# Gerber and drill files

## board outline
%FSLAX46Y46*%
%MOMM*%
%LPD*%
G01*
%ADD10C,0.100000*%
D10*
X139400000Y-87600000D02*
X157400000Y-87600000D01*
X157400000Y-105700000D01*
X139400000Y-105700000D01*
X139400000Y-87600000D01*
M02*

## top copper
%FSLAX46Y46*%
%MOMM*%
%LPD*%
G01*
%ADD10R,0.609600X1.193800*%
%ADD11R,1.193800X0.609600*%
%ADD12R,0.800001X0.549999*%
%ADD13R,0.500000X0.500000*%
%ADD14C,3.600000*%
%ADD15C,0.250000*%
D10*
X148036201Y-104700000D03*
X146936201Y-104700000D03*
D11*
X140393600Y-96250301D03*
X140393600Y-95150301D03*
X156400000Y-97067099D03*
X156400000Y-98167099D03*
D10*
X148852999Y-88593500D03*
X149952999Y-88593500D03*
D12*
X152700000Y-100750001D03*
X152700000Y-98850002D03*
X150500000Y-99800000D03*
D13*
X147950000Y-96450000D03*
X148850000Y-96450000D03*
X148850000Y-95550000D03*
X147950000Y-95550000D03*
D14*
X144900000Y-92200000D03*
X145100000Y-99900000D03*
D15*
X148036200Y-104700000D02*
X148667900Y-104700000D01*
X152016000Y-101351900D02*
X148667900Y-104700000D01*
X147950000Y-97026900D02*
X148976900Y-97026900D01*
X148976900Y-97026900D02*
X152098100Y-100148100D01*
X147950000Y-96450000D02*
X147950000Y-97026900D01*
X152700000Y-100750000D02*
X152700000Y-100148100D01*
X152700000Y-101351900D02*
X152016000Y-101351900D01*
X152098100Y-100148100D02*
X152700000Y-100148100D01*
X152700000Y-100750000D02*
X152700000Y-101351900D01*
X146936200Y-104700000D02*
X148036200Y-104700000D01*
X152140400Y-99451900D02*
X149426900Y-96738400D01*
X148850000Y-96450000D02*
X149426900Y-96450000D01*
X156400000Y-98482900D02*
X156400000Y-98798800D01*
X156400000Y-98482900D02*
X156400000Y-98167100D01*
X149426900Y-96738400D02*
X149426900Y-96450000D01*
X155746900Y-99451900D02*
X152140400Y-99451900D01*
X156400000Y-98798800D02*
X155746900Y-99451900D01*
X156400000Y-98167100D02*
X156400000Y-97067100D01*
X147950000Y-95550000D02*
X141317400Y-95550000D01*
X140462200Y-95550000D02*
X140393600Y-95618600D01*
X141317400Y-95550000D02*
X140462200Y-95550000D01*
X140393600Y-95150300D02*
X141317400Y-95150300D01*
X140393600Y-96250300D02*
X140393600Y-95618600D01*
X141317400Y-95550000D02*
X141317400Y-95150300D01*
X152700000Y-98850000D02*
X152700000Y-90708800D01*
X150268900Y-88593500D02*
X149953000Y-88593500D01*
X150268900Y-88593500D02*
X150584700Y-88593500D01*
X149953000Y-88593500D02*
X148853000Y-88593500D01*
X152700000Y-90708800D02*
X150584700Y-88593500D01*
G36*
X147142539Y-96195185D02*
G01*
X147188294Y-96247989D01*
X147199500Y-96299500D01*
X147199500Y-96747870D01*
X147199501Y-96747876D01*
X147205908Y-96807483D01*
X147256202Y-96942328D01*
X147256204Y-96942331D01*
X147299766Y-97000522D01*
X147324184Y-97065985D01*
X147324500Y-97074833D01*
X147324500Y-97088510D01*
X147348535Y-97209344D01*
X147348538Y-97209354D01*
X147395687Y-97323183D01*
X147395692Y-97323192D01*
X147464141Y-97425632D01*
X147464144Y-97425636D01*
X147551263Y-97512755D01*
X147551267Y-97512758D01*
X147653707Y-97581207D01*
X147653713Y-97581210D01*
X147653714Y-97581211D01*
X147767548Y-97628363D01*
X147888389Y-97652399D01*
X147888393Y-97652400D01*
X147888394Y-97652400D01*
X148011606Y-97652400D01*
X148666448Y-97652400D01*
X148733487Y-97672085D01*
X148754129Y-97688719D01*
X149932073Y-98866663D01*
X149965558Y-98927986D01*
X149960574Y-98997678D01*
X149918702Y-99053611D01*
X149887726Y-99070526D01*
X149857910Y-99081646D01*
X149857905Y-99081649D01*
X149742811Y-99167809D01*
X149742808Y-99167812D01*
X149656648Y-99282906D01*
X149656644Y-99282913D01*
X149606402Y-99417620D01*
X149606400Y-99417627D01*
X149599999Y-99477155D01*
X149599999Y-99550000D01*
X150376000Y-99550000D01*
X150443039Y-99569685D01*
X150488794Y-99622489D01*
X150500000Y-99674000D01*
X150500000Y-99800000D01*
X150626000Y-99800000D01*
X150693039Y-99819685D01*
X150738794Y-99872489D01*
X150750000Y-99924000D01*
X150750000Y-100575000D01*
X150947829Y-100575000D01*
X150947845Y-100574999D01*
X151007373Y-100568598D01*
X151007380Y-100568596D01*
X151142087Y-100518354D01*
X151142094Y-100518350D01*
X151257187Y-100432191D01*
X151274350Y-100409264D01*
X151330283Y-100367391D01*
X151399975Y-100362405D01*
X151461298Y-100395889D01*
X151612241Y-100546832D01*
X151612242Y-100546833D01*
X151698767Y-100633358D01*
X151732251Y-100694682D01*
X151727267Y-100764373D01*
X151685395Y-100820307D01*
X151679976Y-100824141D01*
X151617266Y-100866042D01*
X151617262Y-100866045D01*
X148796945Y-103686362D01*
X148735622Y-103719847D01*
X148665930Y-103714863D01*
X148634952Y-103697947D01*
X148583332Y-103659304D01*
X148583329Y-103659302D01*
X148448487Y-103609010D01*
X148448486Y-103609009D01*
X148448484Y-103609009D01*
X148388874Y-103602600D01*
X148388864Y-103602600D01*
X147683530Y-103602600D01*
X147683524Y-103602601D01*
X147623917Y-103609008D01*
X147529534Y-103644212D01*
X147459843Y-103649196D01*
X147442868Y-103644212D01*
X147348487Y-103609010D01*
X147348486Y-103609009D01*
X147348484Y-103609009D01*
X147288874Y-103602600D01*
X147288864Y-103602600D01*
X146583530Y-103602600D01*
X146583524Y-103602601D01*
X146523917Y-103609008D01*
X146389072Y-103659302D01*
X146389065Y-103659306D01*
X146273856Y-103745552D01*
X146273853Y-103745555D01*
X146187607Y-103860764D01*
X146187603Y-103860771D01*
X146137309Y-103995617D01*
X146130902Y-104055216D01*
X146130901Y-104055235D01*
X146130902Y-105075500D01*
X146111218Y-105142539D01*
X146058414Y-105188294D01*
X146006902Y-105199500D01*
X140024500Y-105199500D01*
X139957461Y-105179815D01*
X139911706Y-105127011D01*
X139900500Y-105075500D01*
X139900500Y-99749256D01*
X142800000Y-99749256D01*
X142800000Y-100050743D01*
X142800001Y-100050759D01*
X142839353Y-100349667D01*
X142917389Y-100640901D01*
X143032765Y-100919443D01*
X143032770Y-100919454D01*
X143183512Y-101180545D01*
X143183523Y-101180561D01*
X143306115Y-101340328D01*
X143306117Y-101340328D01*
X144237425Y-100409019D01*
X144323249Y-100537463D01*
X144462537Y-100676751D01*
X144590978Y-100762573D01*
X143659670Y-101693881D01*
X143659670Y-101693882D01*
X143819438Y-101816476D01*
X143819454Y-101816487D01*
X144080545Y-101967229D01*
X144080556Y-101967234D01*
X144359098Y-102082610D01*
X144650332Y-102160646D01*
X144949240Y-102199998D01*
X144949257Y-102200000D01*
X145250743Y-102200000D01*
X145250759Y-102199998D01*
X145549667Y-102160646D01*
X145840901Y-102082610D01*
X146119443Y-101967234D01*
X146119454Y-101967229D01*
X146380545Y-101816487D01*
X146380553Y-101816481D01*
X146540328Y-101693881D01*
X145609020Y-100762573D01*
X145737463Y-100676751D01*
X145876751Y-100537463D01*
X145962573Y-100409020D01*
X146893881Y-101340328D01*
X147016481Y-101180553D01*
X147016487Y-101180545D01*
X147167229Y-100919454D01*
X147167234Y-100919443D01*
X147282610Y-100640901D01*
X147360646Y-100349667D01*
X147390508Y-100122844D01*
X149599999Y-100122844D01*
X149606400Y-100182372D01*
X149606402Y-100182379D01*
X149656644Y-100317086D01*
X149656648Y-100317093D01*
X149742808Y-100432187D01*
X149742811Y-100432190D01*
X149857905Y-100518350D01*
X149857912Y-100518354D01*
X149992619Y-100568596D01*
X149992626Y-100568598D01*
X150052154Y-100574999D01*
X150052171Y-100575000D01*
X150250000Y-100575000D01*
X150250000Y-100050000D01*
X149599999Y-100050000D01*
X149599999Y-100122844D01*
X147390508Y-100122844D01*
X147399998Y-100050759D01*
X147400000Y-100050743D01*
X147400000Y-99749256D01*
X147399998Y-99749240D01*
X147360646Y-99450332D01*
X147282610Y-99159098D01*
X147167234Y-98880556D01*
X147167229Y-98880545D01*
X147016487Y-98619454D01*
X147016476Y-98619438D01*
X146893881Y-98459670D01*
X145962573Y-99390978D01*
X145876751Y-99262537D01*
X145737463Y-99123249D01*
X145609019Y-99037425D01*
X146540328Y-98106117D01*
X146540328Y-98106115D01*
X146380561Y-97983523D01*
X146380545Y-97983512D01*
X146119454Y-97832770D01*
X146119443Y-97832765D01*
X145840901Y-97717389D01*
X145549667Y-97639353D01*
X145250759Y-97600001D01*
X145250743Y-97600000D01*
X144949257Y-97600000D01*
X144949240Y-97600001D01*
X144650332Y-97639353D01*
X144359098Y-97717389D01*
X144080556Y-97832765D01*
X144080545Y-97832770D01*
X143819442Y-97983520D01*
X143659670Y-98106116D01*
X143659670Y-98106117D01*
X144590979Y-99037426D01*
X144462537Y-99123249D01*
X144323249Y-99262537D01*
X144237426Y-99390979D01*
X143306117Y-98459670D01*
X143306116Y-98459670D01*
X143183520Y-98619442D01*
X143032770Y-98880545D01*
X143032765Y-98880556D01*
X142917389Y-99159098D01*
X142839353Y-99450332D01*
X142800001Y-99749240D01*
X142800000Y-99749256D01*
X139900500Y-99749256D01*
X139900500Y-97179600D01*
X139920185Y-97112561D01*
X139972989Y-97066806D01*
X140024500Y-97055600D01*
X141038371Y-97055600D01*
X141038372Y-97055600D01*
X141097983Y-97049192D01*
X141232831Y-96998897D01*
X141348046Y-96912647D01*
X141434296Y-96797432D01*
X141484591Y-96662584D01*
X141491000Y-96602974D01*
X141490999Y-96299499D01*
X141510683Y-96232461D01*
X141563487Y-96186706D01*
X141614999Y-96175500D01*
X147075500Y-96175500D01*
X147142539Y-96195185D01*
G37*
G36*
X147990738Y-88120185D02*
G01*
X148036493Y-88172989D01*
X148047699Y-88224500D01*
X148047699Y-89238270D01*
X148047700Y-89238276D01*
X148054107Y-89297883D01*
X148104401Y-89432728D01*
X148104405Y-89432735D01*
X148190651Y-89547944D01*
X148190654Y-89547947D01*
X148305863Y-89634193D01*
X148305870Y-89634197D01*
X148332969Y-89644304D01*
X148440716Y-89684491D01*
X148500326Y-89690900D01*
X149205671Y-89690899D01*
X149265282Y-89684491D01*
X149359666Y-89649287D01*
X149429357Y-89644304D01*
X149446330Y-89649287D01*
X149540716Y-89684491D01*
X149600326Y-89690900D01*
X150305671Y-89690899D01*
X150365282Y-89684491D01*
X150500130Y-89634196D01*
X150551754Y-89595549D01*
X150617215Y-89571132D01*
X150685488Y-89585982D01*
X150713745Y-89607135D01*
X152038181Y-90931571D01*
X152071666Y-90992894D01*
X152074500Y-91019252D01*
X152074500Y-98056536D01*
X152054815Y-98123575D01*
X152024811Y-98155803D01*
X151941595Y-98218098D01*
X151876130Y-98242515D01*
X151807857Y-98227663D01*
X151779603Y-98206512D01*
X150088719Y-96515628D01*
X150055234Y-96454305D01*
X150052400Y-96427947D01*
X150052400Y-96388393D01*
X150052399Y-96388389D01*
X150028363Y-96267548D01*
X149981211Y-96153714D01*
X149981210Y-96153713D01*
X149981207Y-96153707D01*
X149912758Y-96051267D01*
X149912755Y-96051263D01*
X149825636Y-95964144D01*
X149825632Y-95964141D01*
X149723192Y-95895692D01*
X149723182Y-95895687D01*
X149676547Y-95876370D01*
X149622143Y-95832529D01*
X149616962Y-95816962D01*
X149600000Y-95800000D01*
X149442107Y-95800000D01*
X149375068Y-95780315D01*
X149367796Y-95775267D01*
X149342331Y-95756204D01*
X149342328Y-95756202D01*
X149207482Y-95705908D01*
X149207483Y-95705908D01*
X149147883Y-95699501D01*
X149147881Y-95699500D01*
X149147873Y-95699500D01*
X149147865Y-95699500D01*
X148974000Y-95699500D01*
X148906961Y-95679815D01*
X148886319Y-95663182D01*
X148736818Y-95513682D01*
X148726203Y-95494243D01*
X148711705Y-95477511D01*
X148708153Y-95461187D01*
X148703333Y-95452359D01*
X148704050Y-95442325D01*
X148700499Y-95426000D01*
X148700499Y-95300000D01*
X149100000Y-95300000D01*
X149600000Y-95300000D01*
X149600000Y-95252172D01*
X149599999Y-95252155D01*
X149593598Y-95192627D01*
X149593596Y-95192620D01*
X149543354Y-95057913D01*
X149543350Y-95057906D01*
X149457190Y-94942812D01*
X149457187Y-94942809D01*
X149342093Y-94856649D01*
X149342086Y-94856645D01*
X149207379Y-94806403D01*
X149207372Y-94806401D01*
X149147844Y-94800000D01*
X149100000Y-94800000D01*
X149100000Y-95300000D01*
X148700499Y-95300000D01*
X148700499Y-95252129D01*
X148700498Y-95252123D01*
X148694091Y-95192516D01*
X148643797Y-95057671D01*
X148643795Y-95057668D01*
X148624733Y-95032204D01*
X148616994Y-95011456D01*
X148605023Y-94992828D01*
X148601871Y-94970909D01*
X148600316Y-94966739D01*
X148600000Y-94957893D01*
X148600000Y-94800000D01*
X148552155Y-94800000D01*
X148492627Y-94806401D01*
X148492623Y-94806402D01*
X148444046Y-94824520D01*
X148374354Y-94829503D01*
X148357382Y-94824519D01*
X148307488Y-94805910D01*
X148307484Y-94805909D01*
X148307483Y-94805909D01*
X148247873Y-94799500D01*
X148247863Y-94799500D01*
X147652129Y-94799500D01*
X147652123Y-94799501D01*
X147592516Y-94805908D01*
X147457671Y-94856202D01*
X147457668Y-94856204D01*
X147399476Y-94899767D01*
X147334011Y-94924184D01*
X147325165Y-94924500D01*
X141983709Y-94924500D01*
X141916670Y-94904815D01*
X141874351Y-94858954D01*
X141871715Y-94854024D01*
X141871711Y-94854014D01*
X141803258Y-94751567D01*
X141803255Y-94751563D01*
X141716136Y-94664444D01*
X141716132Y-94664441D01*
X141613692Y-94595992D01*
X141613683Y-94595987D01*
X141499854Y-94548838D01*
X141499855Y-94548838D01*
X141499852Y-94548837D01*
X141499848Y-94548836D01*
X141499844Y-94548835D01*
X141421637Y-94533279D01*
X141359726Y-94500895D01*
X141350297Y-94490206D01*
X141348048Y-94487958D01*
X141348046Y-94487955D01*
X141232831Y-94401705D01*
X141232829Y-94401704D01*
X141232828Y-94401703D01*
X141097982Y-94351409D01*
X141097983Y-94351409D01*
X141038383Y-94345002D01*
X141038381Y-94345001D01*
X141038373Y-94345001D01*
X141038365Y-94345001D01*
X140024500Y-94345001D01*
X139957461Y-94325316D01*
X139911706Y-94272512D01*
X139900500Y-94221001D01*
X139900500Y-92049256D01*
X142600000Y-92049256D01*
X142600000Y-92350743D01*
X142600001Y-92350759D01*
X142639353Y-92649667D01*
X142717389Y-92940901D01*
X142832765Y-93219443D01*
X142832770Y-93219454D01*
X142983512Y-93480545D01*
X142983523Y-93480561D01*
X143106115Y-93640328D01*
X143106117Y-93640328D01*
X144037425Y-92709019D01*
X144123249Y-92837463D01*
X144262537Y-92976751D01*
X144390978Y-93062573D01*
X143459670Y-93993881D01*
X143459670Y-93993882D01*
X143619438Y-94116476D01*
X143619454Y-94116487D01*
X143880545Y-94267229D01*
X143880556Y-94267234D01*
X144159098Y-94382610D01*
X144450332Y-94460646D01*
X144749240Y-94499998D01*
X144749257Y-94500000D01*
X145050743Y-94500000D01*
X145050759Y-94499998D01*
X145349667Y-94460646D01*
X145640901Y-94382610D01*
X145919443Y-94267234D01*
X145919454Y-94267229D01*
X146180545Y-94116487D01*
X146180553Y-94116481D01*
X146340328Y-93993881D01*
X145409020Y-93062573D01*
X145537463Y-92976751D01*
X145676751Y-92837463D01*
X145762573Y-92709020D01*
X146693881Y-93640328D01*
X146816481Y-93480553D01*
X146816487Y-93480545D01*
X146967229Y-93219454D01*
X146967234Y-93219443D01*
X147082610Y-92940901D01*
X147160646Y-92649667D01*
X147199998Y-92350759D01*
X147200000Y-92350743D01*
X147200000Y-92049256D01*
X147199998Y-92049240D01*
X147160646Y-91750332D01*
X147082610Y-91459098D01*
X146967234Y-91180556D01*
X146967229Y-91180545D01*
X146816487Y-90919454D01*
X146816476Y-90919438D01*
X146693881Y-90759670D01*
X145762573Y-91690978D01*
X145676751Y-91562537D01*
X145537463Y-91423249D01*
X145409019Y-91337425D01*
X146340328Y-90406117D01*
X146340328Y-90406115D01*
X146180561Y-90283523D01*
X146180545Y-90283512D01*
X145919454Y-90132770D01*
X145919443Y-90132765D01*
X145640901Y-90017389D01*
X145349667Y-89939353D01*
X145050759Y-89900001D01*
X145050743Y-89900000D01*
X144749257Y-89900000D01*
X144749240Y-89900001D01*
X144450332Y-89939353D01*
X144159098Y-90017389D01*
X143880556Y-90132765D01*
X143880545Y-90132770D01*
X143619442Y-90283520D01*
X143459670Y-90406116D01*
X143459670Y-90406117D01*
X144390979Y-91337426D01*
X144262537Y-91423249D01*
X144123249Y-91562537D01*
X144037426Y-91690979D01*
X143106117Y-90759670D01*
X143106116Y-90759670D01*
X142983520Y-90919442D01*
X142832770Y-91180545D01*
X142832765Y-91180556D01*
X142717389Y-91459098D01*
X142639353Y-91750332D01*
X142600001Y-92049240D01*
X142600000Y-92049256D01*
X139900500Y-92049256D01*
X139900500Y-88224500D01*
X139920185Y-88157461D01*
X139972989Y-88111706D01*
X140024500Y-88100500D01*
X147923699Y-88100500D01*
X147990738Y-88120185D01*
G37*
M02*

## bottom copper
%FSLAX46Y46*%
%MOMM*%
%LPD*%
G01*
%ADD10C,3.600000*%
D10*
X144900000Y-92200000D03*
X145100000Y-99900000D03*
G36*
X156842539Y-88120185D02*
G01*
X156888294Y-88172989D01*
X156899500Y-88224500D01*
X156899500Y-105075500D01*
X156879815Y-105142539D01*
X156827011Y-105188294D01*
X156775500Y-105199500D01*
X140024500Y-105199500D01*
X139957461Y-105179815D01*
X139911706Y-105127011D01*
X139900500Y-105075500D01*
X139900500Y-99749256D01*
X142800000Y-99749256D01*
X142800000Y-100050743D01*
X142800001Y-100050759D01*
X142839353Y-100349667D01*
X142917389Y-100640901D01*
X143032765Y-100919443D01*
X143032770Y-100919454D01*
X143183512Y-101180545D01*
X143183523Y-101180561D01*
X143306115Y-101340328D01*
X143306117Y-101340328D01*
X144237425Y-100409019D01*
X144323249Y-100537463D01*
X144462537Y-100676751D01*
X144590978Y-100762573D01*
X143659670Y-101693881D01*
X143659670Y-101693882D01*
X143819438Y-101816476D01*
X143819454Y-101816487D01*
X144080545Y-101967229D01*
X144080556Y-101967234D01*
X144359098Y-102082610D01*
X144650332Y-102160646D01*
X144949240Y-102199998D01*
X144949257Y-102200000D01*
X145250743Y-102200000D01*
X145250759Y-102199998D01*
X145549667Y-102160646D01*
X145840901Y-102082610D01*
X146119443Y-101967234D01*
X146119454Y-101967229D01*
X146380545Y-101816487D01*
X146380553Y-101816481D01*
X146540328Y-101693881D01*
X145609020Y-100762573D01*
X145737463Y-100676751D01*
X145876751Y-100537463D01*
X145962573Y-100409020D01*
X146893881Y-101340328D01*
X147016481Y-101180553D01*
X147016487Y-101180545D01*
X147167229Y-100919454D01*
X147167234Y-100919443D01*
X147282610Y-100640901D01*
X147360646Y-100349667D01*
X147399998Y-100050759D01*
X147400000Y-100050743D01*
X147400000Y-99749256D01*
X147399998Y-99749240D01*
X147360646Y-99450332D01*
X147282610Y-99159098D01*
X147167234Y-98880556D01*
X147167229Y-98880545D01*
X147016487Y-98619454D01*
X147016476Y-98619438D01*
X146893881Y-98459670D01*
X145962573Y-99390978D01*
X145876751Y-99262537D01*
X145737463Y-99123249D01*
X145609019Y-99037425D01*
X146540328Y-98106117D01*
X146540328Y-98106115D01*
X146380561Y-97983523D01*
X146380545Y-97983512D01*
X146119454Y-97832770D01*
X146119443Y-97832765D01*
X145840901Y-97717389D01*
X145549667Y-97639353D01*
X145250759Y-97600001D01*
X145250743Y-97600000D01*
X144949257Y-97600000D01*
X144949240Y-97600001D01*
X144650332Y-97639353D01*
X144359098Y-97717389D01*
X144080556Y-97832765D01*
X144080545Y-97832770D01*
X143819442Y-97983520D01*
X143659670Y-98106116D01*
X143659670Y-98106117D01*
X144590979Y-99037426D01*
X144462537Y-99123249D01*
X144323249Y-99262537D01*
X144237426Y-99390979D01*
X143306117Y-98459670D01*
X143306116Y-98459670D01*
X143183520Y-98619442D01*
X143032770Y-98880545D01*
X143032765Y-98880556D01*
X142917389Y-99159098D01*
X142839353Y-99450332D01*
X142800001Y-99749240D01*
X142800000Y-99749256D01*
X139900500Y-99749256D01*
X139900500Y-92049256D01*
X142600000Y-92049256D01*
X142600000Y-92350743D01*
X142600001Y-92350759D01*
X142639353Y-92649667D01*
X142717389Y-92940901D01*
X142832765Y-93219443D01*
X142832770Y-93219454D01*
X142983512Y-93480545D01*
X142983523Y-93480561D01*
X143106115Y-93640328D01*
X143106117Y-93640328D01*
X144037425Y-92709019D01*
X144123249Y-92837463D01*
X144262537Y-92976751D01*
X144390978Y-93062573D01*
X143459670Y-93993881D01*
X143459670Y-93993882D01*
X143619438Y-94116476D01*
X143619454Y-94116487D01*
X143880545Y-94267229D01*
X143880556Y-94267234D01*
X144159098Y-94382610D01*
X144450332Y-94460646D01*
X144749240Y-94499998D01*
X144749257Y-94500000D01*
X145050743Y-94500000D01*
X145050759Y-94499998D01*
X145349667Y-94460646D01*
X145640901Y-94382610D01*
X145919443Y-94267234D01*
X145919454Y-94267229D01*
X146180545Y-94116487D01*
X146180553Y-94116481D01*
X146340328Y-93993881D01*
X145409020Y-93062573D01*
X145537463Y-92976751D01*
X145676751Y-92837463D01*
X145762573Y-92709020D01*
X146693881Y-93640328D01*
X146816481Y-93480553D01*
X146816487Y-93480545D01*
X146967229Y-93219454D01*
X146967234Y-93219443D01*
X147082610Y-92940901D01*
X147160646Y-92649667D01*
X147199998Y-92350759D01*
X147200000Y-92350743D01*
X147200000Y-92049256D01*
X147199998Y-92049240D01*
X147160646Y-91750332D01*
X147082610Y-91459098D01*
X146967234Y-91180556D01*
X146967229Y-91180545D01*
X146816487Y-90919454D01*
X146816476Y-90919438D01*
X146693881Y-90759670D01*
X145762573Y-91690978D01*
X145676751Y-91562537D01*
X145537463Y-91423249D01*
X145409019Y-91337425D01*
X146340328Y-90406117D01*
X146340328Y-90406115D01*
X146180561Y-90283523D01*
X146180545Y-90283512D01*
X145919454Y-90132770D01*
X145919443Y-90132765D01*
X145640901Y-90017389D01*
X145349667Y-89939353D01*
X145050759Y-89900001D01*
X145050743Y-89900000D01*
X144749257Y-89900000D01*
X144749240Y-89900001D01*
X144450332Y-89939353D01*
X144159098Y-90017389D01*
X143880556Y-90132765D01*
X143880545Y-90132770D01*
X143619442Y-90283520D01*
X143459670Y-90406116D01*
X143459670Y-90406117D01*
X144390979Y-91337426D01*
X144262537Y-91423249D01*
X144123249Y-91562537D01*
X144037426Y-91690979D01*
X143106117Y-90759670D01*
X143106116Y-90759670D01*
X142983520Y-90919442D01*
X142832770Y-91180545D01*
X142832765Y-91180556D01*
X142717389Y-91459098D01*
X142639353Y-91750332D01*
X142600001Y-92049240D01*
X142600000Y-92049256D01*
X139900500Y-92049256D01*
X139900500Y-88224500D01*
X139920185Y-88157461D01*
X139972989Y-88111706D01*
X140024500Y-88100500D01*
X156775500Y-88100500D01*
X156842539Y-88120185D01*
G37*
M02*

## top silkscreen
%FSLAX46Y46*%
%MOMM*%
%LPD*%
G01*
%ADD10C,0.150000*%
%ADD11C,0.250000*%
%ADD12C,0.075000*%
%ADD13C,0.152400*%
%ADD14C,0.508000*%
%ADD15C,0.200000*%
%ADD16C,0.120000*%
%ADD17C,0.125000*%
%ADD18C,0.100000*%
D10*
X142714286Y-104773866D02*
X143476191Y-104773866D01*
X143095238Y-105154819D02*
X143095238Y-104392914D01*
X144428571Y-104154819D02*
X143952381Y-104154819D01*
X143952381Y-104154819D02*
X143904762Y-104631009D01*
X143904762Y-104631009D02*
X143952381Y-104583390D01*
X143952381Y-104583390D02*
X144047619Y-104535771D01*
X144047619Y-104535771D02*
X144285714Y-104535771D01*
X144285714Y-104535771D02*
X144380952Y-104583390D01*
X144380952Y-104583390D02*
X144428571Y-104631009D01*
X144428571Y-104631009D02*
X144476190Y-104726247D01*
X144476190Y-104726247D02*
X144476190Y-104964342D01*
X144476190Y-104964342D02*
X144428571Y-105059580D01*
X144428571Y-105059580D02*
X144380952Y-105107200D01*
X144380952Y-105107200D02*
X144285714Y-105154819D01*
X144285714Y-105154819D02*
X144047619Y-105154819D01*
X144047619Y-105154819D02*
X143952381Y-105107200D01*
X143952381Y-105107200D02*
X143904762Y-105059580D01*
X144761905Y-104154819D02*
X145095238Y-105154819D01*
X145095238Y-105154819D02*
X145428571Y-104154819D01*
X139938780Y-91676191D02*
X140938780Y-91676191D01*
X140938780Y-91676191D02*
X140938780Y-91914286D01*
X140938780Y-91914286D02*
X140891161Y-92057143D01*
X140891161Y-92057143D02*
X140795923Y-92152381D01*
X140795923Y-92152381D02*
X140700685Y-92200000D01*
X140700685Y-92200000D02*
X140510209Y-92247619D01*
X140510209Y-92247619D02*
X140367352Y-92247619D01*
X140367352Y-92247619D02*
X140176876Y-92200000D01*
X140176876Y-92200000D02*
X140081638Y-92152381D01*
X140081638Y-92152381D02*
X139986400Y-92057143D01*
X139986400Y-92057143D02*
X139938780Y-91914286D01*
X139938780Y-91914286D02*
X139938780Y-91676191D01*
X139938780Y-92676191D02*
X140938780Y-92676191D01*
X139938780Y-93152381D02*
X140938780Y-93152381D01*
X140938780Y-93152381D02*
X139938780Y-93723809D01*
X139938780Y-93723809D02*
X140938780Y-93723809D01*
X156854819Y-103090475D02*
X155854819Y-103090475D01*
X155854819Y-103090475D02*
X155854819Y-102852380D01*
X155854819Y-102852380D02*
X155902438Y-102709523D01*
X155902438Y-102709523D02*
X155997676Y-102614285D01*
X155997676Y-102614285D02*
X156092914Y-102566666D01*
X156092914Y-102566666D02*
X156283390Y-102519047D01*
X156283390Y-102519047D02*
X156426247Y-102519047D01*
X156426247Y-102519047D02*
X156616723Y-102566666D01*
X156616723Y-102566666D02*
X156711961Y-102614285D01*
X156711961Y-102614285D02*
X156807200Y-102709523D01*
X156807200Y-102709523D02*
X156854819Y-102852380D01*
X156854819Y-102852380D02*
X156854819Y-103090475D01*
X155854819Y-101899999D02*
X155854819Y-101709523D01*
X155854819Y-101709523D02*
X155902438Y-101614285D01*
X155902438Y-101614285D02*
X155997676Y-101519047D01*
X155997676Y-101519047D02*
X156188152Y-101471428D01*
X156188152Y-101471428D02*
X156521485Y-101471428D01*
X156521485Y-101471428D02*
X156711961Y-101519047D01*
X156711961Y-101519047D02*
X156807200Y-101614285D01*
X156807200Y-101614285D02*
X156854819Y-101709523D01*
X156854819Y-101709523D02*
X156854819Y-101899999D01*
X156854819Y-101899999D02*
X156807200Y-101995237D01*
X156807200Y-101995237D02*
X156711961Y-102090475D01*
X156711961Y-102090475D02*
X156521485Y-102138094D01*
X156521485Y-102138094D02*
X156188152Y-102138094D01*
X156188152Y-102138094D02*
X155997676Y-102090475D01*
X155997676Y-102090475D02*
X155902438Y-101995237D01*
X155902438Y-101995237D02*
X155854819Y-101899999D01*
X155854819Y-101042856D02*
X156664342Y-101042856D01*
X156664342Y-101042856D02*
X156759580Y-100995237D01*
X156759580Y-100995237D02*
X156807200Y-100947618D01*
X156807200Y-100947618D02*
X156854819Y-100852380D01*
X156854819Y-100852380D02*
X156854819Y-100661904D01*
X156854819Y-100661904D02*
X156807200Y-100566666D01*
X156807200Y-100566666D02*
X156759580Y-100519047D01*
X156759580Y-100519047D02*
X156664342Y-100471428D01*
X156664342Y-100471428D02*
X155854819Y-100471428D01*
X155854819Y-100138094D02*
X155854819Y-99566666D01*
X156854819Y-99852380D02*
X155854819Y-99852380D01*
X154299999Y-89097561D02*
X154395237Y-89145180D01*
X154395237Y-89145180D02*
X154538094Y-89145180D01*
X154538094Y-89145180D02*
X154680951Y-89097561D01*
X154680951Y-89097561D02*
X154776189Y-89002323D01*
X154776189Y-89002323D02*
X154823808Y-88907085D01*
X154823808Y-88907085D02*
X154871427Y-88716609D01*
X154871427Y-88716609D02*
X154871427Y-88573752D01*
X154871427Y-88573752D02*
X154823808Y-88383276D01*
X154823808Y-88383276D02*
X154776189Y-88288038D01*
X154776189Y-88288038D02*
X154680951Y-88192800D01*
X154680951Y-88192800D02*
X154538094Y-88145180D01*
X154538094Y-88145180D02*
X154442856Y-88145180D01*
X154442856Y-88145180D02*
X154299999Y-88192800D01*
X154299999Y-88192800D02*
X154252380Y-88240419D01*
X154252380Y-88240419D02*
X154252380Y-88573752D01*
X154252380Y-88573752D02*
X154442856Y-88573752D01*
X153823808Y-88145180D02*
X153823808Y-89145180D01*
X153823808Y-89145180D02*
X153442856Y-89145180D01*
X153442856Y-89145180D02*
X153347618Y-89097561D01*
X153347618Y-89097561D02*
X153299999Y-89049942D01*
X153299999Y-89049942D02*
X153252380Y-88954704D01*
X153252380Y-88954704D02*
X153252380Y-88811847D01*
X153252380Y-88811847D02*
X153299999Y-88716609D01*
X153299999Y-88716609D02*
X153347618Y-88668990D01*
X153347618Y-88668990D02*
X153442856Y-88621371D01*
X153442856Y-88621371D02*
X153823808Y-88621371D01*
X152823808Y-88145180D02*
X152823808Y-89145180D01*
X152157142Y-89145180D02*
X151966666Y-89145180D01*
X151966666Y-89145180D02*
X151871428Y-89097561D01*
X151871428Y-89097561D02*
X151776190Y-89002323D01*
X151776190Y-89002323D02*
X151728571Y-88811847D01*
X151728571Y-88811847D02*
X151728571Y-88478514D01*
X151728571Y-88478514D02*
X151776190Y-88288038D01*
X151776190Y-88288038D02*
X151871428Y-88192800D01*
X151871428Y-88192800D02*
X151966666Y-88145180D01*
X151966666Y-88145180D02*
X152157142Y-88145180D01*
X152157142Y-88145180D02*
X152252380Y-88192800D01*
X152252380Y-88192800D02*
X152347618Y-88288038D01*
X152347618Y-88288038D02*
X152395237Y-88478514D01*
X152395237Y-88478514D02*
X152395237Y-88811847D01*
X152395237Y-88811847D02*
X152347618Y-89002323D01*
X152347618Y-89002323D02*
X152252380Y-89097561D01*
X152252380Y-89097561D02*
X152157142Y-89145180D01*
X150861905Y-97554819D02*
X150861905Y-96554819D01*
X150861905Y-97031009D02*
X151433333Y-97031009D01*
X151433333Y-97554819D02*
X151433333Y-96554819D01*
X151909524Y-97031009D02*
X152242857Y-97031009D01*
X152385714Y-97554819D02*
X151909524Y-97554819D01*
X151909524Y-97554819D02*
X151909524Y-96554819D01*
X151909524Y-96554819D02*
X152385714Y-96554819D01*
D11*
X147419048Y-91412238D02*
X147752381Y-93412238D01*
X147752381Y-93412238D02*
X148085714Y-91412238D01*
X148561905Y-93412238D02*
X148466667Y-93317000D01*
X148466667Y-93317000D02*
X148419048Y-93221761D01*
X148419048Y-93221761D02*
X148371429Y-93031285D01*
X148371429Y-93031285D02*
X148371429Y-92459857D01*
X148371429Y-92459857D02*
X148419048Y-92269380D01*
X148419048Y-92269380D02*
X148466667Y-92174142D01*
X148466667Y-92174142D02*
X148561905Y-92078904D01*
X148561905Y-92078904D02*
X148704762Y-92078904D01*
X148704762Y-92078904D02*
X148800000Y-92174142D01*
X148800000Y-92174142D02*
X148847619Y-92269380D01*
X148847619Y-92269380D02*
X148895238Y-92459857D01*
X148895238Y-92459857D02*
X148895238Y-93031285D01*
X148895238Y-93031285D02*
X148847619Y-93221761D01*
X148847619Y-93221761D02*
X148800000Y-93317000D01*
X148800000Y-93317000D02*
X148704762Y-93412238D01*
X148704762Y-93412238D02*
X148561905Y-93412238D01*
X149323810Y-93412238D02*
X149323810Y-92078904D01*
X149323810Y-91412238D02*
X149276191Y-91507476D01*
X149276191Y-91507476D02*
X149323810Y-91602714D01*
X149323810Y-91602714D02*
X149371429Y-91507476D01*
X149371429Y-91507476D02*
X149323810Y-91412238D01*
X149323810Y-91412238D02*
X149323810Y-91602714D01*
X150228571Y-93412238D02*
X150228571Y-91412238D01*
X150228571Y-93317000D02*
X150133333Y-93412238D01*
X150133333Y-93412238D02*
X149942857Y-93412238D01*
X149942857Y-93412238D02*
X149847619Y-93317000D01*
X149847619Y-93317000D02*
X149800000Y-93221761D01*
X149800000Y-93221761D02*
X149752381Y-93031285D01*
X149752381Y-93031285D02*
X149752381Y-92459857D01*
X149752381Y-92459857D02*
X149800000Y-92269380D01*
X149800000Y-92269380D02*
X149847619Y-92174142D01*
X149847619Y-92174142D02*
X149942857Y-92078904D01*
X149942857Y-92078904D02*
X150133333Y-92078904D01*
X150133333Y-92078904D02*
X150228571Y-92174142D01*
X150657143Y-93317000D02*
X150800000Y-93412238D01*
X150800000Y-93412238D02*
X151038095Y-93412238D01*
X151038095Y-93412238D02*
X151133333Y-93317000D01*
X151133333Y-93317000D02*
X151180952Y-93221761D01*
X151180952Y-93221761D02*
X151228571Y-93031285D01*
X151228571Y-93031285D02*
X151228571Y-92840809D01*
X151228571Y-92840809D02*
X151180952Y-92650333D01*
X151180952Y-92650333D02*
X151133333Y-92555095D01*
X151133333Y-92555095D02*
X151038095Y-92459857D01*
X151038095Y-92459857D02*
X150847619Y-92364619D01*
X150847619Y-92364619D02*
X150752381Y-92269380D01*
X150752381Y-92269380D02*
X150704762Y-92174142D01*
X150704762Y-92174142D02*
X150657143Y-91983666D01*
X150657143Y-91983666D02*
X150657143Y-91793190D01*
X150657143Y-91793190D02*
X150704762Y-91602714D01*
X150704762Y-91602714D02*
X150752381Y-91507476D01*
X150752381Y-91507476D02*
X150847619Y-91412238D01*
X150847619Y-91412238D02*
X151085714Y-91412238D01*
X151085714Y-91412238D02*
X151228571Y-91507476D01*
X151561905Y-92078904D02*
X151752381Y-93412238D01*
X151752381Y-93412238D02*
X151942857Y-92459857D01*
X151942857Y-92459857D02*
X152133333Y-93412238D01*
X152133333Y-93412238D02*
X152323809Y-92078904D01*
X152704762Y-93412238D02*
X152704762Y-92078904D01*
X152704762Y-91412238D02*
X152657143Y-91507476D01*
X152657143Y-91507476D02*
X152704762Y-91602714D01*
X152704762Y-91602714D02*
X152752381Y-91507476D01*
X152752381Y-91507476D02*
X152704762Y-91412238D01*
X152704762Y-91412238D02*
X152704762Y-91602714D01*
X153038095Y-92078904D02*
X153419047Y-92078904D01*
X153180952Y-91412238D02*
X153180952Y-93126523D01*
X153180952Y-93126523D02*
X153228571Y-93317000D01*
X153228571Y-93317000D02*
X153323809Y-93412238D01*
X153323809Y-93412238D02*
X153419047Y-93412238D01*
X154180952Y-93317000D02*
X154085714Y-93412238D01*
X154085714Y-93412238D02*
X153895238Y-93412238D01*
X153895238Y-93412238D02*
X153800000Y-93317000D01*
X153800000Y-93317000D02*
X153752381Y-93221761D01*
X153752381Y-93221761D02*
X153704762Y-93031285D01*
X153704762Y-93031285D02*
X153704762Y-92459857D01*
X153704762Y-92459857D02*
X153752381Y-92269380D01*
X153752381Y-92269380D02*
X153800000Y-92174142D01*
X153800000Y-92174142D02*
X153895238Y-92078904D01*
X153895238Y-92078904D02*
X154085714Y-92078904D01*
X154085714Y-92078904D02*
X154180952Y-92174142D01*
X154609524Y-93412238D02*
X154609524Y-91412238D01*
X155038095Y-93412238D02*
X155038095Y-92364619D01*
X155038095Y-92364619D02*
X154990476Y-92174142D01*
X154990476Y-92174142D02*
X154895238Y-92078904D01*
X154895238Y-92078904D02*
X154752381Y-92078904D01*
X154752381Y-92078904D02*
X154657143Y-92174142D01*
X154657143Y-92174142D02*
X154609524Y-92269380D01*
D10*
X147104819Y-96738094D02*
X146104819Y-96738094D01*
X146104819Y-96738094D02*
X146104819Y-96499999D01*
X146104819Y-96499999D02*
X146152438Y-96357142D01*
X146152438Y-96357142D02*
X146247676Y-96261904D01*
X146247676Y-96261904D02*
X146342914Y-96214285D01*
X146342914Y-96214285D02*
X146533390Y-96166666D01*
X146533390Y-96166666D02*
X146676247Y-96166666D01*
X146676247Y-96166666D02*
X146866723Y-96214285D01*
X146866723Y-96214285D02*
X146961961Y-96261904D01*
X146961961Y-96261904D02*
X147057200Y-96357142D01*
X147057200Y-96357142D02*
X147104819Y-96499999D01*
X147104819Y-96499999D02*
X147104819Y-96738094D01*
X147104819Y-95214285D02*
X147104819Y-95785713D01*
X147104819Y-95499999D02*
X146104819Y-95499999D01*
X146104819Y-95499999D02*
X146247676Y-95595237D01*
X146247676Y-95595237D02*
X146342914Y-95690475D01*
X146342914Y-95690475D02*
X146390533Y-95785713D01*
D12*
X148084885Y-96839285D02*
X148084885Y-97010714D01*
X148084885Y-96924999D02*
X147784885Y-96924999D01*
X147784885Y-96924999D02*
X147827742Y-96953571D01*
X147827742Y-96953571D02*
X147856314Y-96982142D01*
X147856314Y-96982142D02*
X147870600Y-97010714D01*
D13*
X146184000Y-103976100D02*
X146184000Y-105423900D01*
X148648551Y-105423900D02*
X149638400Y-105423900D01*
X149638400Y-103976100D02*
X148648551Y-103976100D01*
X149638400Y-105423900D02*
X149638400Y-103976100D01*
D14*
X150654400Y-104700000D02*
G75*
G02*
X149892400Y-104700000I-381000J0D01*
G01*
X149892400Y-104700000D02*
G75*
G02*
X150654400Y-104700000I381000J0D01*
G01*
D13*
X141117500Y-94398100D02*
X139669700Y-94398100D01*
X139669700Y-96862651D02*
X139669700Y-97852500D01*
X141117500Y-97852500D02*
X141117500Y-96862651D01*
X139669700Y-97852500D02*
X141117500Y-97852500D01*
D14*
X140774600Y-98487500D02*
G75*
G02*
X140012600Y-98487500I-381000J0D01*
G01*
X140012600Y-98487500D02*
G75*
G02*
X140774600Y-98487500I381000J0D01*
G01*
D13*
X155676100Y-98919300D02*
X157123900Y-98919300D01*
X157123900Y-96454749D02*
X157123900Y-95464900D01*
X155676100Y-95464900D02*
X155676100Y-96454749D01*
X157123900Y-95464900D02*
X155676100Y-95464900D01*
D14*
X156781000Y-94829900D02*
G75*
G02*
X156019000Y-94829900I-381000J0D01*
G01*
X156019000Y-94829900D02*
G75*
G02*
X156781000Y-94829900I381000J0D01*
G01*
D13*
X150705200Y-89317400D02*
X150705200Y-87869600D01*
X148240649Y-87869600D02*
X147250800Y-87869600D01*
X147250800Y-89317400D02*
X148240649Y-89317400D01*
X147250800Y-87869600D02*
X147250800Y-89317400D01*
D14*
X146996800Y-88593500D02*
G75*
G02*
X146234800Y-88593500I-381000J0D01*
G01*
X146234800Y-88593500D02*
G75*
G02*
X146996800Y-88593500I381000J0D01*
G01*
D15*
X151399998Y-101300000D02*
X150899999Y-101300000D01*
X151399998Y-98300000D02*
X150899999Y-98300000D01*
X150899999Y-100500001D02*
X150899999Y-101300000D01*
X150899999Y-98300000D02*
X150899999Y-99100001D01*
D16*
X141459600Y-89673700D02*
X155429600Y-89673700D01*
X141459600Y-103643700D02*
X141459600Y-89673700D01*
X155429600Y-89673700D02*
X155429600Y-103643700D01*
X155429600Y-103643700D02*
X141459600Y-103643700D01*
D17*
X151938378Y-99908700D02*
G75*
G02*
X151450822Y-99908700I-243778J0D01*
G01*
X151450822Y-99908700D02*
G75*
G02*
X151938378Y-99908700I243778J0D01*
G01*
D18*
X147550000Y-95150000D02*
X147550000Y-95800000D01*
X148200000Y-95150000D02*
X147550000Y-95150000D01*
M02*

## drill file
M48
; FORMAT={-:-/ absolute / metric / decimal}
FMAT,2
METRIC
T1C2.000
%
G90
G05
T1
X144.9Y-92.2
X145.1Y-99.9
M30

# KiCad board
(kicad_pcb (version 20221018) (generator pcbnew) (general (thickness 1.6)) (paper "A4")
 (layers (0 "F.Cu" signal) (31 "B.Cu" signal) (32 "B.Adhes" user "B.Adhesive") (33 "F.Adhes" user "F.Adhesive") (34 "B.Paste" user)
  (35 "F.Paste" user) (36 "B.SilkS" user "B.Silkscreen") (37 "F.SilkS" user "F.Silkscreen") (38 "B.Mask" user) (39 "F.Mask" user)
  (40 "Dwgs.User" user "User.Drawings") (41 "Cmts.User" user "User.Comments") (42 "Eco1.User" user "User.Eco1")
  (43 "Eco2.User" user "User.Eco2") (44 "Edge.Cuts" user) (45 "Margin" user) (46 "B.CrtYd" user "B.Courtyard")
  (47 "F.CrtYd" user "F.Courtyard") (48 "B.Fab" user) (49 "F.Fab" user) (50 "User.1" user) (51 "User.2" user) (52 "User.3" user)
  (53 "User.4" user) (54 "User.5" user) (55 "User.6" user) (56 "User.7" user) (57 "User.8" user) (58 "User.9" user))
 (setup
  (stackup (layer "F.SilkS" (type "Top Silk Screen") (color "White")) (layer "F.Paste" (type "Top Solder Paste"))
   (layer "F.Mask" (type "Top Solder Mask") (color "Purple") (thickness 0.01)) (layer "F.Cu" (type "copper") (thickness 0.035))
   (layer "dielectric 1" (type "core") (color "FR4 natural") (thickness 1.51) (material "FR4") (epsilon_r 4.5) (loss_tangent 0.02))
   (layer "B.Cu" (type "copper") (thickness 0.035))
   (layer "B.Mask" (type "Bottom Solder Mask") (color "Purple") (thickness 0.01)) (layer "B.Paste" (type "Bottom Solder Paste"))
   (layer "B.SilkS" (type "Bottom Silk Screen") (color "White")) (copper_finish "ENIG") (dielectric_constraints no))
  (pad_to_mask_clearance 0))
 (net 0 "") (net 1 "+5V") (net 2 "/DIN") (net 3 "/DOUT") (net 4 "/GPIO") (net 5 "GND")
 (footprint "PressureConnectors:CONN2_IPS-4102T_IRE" (layer "F.Cu") (at 148.0362 104.7)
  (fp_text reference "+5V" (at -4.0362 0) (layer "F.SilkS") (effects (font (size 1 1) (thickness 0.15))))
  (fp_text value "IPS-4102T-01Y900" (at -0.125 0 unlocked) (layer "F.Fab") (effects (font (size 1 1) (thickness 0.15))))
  (fp_line (start -1.8522 -0.7239) (end -1.8522 0.7239) (stroke (width 0.1524) (type solid)) (layer "F.SilkS"))
  (fp_line (start 0.612351 0.7239) (end 1.6022 0.7239) (stroke (width 0.1524) (type solid)) (layer "F.SilkS"))
  (fp_line (start 1.6022 -0.7239) (end 0.612351 -0.7239) (stroke (width 0.1524) (type solid)) (layer "F.SilkS"))
  (fp_line (start 1.6022 0.7239) (end 1.6022 -0.7239) (stroke (width 0.1524) (type solid)) (layer "F.SilkS"))
  (fp_circle (center 2.2372 0) (end 2.6182 0) (stroke (width 0.508) (type solid)) (fill none) (layer "F.SilkS"))
  (pad "1" smd rect (at 0.000001 0) (size 0.6096 1.1938) (layers "F.Cu" "F.Paste" "F.Mask") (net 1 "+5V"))
  (pad "2" smd rect (at -1.099999 0) (size 0.6096 1.1938) (layers "F.Cu" "F.Paste" "F.Mask") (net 1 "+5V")))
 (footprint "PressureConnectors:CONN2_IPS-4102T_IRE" (layer "F.Cu") (at 140.3936 96.2503 -90)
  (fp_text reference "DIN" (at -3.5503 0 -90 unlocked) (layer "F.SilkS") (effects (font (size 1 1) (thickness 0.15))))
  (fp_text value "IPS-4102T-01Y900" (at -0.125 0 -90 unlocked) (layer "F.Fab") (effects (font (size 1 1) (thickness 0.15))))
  (fp_line (start -1.8522 -0.7239) (end -1.8522 0.7239) (stroke (width 0.1524) (type solid)) (layer "F.SilkS"))
  (fp_line (start 0.612351 0.7239) (end 1.6022 0.7239) (stroke (width 0.1524) (type solid)) (layer "F.SilkS"))
  (fp_line (start 1.6022 -0.7239) (end 0.612351 -0.7239) (stroke (width 0.1524) (type solid)) (layer "F.SilkS"))
  (fp_line (start 1.6022 0.7239) (end 1.6022 -0.7239) (stroke (width 0.1524) (type solid)) (layer "F.SilkS"))
  (fp_circle (center 2.2372 0) (end 2.6182 0) (stroke (width 0.508) (type solid)) (fill none) (layer "F.SilkS"))
  (pad "1" smd rect (at 0.000001 0 270) (size 0.6096 1.1938) (layers "F.Cu" "F.Paste" "F.Mask") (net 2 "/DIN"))
  (pad "2" smd rect (at -1.099999 0 270) (size 0.6096 1.1938) (layers "F.Cu" "F.Paste" "F.Mask") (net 2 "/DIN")))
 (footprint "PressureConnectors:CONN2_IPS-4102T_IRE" (layer "F.Cu") (at 156.4 97.0671 90)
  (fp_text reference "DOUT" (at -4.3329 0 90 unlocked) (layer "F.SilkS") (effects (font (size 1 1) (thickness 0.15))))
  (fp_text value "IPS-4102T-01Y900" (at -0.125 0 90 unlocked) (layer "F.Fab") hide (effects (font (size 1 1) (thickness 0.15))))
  (fp_line (start -1.8522 -0.7239) (end -1.8522 0.7239) (stroke (width 0.1524) (type solid)) (layer "F.SilkS"))
  (fp_line (start 0.612351 0.7239) (end 1.6022 0.7239) (stroke (width 0.1524) (type solid)) (layer "F.SilkS"))
  (fp_line (start 1.6022 -0.7239) (end 0.612351 -0.7239) (stroke (width 0.1524) (type solid)) (layer "F.SilkS"))
  (fp_line (start 1.6022 0.7239) (end 1.6022 -0.7239) (stroke (width 0.1524) (type solid)) (layer "F.SilkS"))
  (fp_circle (center 2.2372 0) (end 2.6182 0) (stroke (width 0.508) (type solid)) (fill none) (layer "F.SilkS"))
  (pad "1" smd rect (at 0.000001 0 90) (size 0.6096 1.1938) (layers "F.Cu" "F.Paste" "F.Mask") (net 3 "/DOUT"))
  (pad "2" smd rect (at -1.099999 0 90) (size 0.6096 1.1938) (layers "F.Cu" "F.Paste" "F.Mask") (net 3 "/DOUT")))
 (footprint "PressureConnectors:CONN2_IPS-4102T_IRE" (layer "F.Cu") (at 148.853 88.5935 180)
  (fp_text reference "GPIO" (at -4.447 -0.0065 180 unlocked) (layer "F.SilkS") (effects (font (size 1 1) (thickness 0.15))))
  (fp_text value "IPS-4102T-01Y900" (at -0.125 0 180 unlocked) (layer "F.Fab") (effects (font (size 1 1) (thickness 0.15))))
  (fp_line (start -1.8522 -0.7239) (end -1.8522 0.7239) (stroke (width 0.1524) (type solid)) (layer "F.SilkS"))
  (fp_line (start 0.612351 0.7239) (end 1.6022 0.7239) (stroke (width 0.1524) (type solid)) (layer "F.SilkS"))
  (fp_line (start 1.6022 -0.7239) (end 0.612351 -0.7239) (stroke (width 0.1524) (type solid)) (layer "F.SilkS"))
  (fp_line (start 1.6022 0.7239) (end 1.6022 -0.7239) (stroke (width 0.1524) (type solid)) (layer "F.SilkS"))
  (fp_circle (center 2.2372 0) (end 2.6182 0) (stroke (width 0.508) (type solid)) (fill none) (layer "F.SilkS"))
  (pad "1" smd rect (at 0.000001 0 180) (size 0.6096 1.1938) (layers "F.Cu" "F.Paste" "F.Mask") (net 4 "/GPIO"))
  (pad "2" smd rect (at -1.099999 0 180) (size 0.6096 1.1938) (layers "F.Cu" "F.Paste" "F.Mask") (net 4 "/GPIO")))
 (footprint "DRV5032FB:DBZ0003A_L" (layer "F.Cu") (at 151.6 99.8 180)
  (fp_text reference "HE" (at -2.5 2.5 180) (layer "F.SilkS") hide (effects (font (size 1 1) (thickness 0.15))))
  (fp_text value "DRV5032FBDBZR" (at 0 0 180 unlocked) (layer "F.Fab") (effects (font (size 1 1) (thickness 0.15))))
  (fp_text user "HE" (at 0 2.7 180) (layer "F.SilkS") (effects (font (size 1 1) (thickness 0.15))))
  (fp_line (start 0.200002 -1.5) (end 0.700001 -1.5) (stroke (width 0.2) (type solid)) (layer "F.SilkS"))
  (fp_line (start 0.200002 1.5) (end 0.700001 1.5) (stroke (width 0.2) (type solid)) (layer "F.SilkS"))
  (fp_line (start 0.700001 -0.700001) (end 0.700001 -1.5) (stroke (width 0.2) (type solid)) (layer "F.SilkS"))
  (fp_line (start 0.700001 1.5) (end 0.700001 0.699999) (stroke (width 0.2) (type solid)) (layer "F.SilkS"))
  (pad "1" smd rect (at -1.1 -0.950001 270) (size 0.549999 0.800001) (layers "F.Cu" "F.Paste" "F.Mask") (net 1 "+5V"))
  (pad "2" smd rect (at -1.1 0.949998 270) (size 0.549999 0.800001) (layers "F.Cu" "F.Paste" "F.Mask") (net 4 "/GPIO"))
  (pad "3" smd rect (at 1.1 0 270) (size 0.549999 0.800001) (layers "F.Cu" "F.Paste" "F.Mask") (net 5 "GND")))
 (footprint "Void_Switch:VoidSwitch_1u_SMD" (layer "F.Cu") (at 148.4446 96.6587)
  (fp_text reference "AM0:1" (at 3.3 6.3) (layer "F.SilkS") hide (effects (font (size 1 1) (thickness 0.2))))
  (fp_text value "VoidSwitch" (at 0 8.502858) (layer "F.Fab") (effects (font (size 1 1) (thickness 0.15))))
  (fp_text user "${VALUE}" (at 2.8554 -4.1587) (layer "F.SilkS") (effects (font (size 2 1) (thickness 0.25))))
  (fp_line (start -6.985 -6.985) (end 6.985 -6.985) (stroke (width 0.12) (type solid)) (layer "F.SilkS"))
  (fp_line (start -6.985 6.985) (end -6.985 -6.985) (stroke (width 0.12) (type solid)) (layer "F.SilkS"))
  (fp_line (start 6.985 -6.985) (end 6.985 6.985) (stroke (width 0.12) (type solid)) (layer "F.SilkS"))
  (fp_line (start 6.985 6.985) (end -6.985 6.985) (stroke (width 0.12) (type solid)) (layer "F.SilkS"))
  (fp_circle (center 3.25 3.25) (end 3.493778 3.25) (stroke (width 0.125) (type solid)) (fill none) (layer "F.SilkS")))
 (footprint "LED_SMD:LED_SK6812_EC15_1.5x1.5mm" (layer "F.Cu") (at 148.4 96 90)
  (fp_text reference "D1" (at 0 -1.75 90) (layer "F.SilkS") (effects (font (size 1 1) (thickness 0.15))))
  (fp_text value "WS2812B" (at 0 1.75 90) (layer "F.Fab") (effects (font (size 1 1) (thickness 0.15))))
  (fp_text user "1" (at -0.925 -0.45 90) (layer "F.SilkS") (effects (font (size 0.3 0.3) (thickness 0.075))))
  (fp_line (start 0.85 -0.85) (end 0.2 -0.85) (stroke (width 0.1) (type solid)) (layer "F.SilkS"))
  (fp_line (start 0.85 -0.2) (end 0.85 -0.85) (stroke (width 0.1) (type solid)) (layer "F.SilkS"))
  (pad "1" smd rect (at -0.45 -0.45 90) (size 0.5 0.5) (layers "F.Cu" "F.Paste" "F.Mask") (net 1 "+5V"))
  (pad "2" smd rect (at -0.45 0.45 90) (size 0.5 0.5) (layers "F.Cu" "F.Paste" "F.Mask") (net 3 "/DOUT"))
  (pad "3" smd rect (at 0.45 0.45 90) (size 0.5 0.5) (layers "F.Cu" "F.Paste" "F.Mask") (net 5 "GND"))
  (pad "4" smd rect (at 0.45 -0.45 90) (size 0.5 0.5) (layers "F.Cu" "F.Paste" "F.Mask") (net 2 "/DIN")))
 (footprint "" (layer "F.Cu") (at 144.9 92.2)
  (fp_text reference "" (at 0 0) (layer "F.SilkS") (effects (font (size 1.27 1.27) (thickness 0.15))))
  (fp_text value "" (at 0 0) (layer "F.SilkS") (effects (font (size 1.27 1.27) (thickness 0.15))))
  (pad "1" thru_hole circle (at 0 0 180) (size 3.6 3.6) (drill 2) (layers "*.Cu" "*.Mask") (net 5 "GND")))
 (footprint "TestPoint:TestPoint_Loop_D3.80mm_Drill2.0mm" (layer "B.Cu") (at 145.1 99.9 180)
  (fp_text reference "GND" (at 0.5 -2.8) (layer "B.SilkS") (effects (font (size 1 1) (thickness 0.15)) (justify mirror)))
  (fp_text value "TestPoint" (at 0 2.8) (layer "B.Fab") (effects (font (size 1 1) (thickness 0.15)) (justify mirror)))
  (pad "1" thru_hole circle (at 0 0 180) (size 3.6 3.6) (drill 2) (layers "*.Cu" "*.Mask") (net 5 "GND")))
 (gr_rect (start 139.4 87.6) (end 157.4 105.7) (stroke (width 0.1) (type default)) (fill none) (layer "Edge.Cuts"))
 (segment (start 148.0362 104.7) (end 148.6679 104.7) (width 0.25) (layer "F.Cu") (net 1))
 (segment (start 152.016 101.3519) (end 148.6679 104.7) (width 0.25) (layer "F.Cu") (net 1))
 (segment (start 147.95 97.0269) (end 148.9769 97.0269) (width 0.25) (layer "F.Cu") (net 1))
 (segment (start 148.9769 97.0269) (end 152.0981 100.1481) (width 0.25) (layer "F.Cu") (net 1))
 (segment (start 147.95 96.45) (end 147.95 97.0269) (width 0.25) (layer "F.Cu") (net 1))
 (segment (start 152.7 100.75) (end 152.7 100.1481) (width 0.25) (layer "F.Cu") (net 1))
 (segment (start 152.7 101.3519) (end 152.016 101.3519) (width 0.25) (layer "F.Cu") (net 1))
 (segment (start 152.0981 100.1481) (end 152.7 100.1481) (width 0.25) (layer "F.Cu") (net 1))
 (segment (start 152.7 100.75) (end 152.7 101.3519) (width 0.25) (layer "F.Cu") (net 1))
 (segment (start 146.9362 104.7) (end 148.0362 104.7) (width 0.25) (layer "F.Cu") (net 1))
 (segment (start 152.1404 99.4519) (end 149.4269 96.7384) (width 0.25) (layer "F.Cu") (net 3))
 (segment (start 148.85 96.45) (end 149.4269 96.45) (width 0.25) (layer "F.Cu") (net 3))
 (segment (start 156.4 98.4829) (end 156.4 98.7988) (width 0.25) (layer "F.Cu") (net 3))
 (segment (start 156.4 98.4829) (end 156.4 98.1671) (width 0.25) (layer "F.Cu") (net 3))
 (segment (start 149.4269 96.7384) (end 149.4269 96.45) (width 0.25) (layer "F.Cu") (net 3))
 (segment (start 155.7469 99.4519) (end 152.1404 99.4519) (width 0.25) (layer "F.Cu") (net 3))
 (segment (start 156.4 98.7988) (end 155.7469 99.4519) (width 0.25) (layer "F.Cu") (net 3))
 (segment (start 156.4 98.1671) (end 156.4 97.0671) (width 0.25) (layer "F.Cu") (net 3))
 (segment (start 147.95 95.55) (end 141.3174 95.55) (width 0.25) (layer "F.Cu") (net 2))
 (segment (start 140.4622 95.55) (end 140.3936 95.6186) (width 0.25) (layer "F.Cu") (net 2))
 (segment (start 141.3174 95.55) (end 140.4622 95.55) (width 0.25) (layer "F.Cu") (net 2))
 (segment (start 140.3936 95.1503) (end 141.3174 95.1503) (width 0.25) (layer "F.Cu") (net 2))
 (segment (start 140.3936 96.2503) (end 140.3936 95.6186) (width 0.25) (layer "F.Cu") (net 2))
 (segment (start 141.3174 95.55) (end 141.3174 95.1503) (width 0.25) (layer "F.Cu") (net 2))
 (segment (start 152.7 98.85) (end 152.7 90.7088) (width 0.25) (layer "F.Cu") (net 4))
 (segment (start 150.2689 88.5935) (end 149.953 88.5935) (width 0.25) (layer "F.Cu") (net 4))
 (segment (start 150.2689 88.5935) (end 150.5847 88.5935) (width 0.25) (layer "F.Cu") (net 4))
 (segment (start 149.953 88.5935) (end 148.853 88.5935) (width 0.25) (layer "F.Cu") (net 4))
 (segment (start 152.7 90.7088) (end 150.5847 88.5935) (width 0.25) (layer "F.Cu") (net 4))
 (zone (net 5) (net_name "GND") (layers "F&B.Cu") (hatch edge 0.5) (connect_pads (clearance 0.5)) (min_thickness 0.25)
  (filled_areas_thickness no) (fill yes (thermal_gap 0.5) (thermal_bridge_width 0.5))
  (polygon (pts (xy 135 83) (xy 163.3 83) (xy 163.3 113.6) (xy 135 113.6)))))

